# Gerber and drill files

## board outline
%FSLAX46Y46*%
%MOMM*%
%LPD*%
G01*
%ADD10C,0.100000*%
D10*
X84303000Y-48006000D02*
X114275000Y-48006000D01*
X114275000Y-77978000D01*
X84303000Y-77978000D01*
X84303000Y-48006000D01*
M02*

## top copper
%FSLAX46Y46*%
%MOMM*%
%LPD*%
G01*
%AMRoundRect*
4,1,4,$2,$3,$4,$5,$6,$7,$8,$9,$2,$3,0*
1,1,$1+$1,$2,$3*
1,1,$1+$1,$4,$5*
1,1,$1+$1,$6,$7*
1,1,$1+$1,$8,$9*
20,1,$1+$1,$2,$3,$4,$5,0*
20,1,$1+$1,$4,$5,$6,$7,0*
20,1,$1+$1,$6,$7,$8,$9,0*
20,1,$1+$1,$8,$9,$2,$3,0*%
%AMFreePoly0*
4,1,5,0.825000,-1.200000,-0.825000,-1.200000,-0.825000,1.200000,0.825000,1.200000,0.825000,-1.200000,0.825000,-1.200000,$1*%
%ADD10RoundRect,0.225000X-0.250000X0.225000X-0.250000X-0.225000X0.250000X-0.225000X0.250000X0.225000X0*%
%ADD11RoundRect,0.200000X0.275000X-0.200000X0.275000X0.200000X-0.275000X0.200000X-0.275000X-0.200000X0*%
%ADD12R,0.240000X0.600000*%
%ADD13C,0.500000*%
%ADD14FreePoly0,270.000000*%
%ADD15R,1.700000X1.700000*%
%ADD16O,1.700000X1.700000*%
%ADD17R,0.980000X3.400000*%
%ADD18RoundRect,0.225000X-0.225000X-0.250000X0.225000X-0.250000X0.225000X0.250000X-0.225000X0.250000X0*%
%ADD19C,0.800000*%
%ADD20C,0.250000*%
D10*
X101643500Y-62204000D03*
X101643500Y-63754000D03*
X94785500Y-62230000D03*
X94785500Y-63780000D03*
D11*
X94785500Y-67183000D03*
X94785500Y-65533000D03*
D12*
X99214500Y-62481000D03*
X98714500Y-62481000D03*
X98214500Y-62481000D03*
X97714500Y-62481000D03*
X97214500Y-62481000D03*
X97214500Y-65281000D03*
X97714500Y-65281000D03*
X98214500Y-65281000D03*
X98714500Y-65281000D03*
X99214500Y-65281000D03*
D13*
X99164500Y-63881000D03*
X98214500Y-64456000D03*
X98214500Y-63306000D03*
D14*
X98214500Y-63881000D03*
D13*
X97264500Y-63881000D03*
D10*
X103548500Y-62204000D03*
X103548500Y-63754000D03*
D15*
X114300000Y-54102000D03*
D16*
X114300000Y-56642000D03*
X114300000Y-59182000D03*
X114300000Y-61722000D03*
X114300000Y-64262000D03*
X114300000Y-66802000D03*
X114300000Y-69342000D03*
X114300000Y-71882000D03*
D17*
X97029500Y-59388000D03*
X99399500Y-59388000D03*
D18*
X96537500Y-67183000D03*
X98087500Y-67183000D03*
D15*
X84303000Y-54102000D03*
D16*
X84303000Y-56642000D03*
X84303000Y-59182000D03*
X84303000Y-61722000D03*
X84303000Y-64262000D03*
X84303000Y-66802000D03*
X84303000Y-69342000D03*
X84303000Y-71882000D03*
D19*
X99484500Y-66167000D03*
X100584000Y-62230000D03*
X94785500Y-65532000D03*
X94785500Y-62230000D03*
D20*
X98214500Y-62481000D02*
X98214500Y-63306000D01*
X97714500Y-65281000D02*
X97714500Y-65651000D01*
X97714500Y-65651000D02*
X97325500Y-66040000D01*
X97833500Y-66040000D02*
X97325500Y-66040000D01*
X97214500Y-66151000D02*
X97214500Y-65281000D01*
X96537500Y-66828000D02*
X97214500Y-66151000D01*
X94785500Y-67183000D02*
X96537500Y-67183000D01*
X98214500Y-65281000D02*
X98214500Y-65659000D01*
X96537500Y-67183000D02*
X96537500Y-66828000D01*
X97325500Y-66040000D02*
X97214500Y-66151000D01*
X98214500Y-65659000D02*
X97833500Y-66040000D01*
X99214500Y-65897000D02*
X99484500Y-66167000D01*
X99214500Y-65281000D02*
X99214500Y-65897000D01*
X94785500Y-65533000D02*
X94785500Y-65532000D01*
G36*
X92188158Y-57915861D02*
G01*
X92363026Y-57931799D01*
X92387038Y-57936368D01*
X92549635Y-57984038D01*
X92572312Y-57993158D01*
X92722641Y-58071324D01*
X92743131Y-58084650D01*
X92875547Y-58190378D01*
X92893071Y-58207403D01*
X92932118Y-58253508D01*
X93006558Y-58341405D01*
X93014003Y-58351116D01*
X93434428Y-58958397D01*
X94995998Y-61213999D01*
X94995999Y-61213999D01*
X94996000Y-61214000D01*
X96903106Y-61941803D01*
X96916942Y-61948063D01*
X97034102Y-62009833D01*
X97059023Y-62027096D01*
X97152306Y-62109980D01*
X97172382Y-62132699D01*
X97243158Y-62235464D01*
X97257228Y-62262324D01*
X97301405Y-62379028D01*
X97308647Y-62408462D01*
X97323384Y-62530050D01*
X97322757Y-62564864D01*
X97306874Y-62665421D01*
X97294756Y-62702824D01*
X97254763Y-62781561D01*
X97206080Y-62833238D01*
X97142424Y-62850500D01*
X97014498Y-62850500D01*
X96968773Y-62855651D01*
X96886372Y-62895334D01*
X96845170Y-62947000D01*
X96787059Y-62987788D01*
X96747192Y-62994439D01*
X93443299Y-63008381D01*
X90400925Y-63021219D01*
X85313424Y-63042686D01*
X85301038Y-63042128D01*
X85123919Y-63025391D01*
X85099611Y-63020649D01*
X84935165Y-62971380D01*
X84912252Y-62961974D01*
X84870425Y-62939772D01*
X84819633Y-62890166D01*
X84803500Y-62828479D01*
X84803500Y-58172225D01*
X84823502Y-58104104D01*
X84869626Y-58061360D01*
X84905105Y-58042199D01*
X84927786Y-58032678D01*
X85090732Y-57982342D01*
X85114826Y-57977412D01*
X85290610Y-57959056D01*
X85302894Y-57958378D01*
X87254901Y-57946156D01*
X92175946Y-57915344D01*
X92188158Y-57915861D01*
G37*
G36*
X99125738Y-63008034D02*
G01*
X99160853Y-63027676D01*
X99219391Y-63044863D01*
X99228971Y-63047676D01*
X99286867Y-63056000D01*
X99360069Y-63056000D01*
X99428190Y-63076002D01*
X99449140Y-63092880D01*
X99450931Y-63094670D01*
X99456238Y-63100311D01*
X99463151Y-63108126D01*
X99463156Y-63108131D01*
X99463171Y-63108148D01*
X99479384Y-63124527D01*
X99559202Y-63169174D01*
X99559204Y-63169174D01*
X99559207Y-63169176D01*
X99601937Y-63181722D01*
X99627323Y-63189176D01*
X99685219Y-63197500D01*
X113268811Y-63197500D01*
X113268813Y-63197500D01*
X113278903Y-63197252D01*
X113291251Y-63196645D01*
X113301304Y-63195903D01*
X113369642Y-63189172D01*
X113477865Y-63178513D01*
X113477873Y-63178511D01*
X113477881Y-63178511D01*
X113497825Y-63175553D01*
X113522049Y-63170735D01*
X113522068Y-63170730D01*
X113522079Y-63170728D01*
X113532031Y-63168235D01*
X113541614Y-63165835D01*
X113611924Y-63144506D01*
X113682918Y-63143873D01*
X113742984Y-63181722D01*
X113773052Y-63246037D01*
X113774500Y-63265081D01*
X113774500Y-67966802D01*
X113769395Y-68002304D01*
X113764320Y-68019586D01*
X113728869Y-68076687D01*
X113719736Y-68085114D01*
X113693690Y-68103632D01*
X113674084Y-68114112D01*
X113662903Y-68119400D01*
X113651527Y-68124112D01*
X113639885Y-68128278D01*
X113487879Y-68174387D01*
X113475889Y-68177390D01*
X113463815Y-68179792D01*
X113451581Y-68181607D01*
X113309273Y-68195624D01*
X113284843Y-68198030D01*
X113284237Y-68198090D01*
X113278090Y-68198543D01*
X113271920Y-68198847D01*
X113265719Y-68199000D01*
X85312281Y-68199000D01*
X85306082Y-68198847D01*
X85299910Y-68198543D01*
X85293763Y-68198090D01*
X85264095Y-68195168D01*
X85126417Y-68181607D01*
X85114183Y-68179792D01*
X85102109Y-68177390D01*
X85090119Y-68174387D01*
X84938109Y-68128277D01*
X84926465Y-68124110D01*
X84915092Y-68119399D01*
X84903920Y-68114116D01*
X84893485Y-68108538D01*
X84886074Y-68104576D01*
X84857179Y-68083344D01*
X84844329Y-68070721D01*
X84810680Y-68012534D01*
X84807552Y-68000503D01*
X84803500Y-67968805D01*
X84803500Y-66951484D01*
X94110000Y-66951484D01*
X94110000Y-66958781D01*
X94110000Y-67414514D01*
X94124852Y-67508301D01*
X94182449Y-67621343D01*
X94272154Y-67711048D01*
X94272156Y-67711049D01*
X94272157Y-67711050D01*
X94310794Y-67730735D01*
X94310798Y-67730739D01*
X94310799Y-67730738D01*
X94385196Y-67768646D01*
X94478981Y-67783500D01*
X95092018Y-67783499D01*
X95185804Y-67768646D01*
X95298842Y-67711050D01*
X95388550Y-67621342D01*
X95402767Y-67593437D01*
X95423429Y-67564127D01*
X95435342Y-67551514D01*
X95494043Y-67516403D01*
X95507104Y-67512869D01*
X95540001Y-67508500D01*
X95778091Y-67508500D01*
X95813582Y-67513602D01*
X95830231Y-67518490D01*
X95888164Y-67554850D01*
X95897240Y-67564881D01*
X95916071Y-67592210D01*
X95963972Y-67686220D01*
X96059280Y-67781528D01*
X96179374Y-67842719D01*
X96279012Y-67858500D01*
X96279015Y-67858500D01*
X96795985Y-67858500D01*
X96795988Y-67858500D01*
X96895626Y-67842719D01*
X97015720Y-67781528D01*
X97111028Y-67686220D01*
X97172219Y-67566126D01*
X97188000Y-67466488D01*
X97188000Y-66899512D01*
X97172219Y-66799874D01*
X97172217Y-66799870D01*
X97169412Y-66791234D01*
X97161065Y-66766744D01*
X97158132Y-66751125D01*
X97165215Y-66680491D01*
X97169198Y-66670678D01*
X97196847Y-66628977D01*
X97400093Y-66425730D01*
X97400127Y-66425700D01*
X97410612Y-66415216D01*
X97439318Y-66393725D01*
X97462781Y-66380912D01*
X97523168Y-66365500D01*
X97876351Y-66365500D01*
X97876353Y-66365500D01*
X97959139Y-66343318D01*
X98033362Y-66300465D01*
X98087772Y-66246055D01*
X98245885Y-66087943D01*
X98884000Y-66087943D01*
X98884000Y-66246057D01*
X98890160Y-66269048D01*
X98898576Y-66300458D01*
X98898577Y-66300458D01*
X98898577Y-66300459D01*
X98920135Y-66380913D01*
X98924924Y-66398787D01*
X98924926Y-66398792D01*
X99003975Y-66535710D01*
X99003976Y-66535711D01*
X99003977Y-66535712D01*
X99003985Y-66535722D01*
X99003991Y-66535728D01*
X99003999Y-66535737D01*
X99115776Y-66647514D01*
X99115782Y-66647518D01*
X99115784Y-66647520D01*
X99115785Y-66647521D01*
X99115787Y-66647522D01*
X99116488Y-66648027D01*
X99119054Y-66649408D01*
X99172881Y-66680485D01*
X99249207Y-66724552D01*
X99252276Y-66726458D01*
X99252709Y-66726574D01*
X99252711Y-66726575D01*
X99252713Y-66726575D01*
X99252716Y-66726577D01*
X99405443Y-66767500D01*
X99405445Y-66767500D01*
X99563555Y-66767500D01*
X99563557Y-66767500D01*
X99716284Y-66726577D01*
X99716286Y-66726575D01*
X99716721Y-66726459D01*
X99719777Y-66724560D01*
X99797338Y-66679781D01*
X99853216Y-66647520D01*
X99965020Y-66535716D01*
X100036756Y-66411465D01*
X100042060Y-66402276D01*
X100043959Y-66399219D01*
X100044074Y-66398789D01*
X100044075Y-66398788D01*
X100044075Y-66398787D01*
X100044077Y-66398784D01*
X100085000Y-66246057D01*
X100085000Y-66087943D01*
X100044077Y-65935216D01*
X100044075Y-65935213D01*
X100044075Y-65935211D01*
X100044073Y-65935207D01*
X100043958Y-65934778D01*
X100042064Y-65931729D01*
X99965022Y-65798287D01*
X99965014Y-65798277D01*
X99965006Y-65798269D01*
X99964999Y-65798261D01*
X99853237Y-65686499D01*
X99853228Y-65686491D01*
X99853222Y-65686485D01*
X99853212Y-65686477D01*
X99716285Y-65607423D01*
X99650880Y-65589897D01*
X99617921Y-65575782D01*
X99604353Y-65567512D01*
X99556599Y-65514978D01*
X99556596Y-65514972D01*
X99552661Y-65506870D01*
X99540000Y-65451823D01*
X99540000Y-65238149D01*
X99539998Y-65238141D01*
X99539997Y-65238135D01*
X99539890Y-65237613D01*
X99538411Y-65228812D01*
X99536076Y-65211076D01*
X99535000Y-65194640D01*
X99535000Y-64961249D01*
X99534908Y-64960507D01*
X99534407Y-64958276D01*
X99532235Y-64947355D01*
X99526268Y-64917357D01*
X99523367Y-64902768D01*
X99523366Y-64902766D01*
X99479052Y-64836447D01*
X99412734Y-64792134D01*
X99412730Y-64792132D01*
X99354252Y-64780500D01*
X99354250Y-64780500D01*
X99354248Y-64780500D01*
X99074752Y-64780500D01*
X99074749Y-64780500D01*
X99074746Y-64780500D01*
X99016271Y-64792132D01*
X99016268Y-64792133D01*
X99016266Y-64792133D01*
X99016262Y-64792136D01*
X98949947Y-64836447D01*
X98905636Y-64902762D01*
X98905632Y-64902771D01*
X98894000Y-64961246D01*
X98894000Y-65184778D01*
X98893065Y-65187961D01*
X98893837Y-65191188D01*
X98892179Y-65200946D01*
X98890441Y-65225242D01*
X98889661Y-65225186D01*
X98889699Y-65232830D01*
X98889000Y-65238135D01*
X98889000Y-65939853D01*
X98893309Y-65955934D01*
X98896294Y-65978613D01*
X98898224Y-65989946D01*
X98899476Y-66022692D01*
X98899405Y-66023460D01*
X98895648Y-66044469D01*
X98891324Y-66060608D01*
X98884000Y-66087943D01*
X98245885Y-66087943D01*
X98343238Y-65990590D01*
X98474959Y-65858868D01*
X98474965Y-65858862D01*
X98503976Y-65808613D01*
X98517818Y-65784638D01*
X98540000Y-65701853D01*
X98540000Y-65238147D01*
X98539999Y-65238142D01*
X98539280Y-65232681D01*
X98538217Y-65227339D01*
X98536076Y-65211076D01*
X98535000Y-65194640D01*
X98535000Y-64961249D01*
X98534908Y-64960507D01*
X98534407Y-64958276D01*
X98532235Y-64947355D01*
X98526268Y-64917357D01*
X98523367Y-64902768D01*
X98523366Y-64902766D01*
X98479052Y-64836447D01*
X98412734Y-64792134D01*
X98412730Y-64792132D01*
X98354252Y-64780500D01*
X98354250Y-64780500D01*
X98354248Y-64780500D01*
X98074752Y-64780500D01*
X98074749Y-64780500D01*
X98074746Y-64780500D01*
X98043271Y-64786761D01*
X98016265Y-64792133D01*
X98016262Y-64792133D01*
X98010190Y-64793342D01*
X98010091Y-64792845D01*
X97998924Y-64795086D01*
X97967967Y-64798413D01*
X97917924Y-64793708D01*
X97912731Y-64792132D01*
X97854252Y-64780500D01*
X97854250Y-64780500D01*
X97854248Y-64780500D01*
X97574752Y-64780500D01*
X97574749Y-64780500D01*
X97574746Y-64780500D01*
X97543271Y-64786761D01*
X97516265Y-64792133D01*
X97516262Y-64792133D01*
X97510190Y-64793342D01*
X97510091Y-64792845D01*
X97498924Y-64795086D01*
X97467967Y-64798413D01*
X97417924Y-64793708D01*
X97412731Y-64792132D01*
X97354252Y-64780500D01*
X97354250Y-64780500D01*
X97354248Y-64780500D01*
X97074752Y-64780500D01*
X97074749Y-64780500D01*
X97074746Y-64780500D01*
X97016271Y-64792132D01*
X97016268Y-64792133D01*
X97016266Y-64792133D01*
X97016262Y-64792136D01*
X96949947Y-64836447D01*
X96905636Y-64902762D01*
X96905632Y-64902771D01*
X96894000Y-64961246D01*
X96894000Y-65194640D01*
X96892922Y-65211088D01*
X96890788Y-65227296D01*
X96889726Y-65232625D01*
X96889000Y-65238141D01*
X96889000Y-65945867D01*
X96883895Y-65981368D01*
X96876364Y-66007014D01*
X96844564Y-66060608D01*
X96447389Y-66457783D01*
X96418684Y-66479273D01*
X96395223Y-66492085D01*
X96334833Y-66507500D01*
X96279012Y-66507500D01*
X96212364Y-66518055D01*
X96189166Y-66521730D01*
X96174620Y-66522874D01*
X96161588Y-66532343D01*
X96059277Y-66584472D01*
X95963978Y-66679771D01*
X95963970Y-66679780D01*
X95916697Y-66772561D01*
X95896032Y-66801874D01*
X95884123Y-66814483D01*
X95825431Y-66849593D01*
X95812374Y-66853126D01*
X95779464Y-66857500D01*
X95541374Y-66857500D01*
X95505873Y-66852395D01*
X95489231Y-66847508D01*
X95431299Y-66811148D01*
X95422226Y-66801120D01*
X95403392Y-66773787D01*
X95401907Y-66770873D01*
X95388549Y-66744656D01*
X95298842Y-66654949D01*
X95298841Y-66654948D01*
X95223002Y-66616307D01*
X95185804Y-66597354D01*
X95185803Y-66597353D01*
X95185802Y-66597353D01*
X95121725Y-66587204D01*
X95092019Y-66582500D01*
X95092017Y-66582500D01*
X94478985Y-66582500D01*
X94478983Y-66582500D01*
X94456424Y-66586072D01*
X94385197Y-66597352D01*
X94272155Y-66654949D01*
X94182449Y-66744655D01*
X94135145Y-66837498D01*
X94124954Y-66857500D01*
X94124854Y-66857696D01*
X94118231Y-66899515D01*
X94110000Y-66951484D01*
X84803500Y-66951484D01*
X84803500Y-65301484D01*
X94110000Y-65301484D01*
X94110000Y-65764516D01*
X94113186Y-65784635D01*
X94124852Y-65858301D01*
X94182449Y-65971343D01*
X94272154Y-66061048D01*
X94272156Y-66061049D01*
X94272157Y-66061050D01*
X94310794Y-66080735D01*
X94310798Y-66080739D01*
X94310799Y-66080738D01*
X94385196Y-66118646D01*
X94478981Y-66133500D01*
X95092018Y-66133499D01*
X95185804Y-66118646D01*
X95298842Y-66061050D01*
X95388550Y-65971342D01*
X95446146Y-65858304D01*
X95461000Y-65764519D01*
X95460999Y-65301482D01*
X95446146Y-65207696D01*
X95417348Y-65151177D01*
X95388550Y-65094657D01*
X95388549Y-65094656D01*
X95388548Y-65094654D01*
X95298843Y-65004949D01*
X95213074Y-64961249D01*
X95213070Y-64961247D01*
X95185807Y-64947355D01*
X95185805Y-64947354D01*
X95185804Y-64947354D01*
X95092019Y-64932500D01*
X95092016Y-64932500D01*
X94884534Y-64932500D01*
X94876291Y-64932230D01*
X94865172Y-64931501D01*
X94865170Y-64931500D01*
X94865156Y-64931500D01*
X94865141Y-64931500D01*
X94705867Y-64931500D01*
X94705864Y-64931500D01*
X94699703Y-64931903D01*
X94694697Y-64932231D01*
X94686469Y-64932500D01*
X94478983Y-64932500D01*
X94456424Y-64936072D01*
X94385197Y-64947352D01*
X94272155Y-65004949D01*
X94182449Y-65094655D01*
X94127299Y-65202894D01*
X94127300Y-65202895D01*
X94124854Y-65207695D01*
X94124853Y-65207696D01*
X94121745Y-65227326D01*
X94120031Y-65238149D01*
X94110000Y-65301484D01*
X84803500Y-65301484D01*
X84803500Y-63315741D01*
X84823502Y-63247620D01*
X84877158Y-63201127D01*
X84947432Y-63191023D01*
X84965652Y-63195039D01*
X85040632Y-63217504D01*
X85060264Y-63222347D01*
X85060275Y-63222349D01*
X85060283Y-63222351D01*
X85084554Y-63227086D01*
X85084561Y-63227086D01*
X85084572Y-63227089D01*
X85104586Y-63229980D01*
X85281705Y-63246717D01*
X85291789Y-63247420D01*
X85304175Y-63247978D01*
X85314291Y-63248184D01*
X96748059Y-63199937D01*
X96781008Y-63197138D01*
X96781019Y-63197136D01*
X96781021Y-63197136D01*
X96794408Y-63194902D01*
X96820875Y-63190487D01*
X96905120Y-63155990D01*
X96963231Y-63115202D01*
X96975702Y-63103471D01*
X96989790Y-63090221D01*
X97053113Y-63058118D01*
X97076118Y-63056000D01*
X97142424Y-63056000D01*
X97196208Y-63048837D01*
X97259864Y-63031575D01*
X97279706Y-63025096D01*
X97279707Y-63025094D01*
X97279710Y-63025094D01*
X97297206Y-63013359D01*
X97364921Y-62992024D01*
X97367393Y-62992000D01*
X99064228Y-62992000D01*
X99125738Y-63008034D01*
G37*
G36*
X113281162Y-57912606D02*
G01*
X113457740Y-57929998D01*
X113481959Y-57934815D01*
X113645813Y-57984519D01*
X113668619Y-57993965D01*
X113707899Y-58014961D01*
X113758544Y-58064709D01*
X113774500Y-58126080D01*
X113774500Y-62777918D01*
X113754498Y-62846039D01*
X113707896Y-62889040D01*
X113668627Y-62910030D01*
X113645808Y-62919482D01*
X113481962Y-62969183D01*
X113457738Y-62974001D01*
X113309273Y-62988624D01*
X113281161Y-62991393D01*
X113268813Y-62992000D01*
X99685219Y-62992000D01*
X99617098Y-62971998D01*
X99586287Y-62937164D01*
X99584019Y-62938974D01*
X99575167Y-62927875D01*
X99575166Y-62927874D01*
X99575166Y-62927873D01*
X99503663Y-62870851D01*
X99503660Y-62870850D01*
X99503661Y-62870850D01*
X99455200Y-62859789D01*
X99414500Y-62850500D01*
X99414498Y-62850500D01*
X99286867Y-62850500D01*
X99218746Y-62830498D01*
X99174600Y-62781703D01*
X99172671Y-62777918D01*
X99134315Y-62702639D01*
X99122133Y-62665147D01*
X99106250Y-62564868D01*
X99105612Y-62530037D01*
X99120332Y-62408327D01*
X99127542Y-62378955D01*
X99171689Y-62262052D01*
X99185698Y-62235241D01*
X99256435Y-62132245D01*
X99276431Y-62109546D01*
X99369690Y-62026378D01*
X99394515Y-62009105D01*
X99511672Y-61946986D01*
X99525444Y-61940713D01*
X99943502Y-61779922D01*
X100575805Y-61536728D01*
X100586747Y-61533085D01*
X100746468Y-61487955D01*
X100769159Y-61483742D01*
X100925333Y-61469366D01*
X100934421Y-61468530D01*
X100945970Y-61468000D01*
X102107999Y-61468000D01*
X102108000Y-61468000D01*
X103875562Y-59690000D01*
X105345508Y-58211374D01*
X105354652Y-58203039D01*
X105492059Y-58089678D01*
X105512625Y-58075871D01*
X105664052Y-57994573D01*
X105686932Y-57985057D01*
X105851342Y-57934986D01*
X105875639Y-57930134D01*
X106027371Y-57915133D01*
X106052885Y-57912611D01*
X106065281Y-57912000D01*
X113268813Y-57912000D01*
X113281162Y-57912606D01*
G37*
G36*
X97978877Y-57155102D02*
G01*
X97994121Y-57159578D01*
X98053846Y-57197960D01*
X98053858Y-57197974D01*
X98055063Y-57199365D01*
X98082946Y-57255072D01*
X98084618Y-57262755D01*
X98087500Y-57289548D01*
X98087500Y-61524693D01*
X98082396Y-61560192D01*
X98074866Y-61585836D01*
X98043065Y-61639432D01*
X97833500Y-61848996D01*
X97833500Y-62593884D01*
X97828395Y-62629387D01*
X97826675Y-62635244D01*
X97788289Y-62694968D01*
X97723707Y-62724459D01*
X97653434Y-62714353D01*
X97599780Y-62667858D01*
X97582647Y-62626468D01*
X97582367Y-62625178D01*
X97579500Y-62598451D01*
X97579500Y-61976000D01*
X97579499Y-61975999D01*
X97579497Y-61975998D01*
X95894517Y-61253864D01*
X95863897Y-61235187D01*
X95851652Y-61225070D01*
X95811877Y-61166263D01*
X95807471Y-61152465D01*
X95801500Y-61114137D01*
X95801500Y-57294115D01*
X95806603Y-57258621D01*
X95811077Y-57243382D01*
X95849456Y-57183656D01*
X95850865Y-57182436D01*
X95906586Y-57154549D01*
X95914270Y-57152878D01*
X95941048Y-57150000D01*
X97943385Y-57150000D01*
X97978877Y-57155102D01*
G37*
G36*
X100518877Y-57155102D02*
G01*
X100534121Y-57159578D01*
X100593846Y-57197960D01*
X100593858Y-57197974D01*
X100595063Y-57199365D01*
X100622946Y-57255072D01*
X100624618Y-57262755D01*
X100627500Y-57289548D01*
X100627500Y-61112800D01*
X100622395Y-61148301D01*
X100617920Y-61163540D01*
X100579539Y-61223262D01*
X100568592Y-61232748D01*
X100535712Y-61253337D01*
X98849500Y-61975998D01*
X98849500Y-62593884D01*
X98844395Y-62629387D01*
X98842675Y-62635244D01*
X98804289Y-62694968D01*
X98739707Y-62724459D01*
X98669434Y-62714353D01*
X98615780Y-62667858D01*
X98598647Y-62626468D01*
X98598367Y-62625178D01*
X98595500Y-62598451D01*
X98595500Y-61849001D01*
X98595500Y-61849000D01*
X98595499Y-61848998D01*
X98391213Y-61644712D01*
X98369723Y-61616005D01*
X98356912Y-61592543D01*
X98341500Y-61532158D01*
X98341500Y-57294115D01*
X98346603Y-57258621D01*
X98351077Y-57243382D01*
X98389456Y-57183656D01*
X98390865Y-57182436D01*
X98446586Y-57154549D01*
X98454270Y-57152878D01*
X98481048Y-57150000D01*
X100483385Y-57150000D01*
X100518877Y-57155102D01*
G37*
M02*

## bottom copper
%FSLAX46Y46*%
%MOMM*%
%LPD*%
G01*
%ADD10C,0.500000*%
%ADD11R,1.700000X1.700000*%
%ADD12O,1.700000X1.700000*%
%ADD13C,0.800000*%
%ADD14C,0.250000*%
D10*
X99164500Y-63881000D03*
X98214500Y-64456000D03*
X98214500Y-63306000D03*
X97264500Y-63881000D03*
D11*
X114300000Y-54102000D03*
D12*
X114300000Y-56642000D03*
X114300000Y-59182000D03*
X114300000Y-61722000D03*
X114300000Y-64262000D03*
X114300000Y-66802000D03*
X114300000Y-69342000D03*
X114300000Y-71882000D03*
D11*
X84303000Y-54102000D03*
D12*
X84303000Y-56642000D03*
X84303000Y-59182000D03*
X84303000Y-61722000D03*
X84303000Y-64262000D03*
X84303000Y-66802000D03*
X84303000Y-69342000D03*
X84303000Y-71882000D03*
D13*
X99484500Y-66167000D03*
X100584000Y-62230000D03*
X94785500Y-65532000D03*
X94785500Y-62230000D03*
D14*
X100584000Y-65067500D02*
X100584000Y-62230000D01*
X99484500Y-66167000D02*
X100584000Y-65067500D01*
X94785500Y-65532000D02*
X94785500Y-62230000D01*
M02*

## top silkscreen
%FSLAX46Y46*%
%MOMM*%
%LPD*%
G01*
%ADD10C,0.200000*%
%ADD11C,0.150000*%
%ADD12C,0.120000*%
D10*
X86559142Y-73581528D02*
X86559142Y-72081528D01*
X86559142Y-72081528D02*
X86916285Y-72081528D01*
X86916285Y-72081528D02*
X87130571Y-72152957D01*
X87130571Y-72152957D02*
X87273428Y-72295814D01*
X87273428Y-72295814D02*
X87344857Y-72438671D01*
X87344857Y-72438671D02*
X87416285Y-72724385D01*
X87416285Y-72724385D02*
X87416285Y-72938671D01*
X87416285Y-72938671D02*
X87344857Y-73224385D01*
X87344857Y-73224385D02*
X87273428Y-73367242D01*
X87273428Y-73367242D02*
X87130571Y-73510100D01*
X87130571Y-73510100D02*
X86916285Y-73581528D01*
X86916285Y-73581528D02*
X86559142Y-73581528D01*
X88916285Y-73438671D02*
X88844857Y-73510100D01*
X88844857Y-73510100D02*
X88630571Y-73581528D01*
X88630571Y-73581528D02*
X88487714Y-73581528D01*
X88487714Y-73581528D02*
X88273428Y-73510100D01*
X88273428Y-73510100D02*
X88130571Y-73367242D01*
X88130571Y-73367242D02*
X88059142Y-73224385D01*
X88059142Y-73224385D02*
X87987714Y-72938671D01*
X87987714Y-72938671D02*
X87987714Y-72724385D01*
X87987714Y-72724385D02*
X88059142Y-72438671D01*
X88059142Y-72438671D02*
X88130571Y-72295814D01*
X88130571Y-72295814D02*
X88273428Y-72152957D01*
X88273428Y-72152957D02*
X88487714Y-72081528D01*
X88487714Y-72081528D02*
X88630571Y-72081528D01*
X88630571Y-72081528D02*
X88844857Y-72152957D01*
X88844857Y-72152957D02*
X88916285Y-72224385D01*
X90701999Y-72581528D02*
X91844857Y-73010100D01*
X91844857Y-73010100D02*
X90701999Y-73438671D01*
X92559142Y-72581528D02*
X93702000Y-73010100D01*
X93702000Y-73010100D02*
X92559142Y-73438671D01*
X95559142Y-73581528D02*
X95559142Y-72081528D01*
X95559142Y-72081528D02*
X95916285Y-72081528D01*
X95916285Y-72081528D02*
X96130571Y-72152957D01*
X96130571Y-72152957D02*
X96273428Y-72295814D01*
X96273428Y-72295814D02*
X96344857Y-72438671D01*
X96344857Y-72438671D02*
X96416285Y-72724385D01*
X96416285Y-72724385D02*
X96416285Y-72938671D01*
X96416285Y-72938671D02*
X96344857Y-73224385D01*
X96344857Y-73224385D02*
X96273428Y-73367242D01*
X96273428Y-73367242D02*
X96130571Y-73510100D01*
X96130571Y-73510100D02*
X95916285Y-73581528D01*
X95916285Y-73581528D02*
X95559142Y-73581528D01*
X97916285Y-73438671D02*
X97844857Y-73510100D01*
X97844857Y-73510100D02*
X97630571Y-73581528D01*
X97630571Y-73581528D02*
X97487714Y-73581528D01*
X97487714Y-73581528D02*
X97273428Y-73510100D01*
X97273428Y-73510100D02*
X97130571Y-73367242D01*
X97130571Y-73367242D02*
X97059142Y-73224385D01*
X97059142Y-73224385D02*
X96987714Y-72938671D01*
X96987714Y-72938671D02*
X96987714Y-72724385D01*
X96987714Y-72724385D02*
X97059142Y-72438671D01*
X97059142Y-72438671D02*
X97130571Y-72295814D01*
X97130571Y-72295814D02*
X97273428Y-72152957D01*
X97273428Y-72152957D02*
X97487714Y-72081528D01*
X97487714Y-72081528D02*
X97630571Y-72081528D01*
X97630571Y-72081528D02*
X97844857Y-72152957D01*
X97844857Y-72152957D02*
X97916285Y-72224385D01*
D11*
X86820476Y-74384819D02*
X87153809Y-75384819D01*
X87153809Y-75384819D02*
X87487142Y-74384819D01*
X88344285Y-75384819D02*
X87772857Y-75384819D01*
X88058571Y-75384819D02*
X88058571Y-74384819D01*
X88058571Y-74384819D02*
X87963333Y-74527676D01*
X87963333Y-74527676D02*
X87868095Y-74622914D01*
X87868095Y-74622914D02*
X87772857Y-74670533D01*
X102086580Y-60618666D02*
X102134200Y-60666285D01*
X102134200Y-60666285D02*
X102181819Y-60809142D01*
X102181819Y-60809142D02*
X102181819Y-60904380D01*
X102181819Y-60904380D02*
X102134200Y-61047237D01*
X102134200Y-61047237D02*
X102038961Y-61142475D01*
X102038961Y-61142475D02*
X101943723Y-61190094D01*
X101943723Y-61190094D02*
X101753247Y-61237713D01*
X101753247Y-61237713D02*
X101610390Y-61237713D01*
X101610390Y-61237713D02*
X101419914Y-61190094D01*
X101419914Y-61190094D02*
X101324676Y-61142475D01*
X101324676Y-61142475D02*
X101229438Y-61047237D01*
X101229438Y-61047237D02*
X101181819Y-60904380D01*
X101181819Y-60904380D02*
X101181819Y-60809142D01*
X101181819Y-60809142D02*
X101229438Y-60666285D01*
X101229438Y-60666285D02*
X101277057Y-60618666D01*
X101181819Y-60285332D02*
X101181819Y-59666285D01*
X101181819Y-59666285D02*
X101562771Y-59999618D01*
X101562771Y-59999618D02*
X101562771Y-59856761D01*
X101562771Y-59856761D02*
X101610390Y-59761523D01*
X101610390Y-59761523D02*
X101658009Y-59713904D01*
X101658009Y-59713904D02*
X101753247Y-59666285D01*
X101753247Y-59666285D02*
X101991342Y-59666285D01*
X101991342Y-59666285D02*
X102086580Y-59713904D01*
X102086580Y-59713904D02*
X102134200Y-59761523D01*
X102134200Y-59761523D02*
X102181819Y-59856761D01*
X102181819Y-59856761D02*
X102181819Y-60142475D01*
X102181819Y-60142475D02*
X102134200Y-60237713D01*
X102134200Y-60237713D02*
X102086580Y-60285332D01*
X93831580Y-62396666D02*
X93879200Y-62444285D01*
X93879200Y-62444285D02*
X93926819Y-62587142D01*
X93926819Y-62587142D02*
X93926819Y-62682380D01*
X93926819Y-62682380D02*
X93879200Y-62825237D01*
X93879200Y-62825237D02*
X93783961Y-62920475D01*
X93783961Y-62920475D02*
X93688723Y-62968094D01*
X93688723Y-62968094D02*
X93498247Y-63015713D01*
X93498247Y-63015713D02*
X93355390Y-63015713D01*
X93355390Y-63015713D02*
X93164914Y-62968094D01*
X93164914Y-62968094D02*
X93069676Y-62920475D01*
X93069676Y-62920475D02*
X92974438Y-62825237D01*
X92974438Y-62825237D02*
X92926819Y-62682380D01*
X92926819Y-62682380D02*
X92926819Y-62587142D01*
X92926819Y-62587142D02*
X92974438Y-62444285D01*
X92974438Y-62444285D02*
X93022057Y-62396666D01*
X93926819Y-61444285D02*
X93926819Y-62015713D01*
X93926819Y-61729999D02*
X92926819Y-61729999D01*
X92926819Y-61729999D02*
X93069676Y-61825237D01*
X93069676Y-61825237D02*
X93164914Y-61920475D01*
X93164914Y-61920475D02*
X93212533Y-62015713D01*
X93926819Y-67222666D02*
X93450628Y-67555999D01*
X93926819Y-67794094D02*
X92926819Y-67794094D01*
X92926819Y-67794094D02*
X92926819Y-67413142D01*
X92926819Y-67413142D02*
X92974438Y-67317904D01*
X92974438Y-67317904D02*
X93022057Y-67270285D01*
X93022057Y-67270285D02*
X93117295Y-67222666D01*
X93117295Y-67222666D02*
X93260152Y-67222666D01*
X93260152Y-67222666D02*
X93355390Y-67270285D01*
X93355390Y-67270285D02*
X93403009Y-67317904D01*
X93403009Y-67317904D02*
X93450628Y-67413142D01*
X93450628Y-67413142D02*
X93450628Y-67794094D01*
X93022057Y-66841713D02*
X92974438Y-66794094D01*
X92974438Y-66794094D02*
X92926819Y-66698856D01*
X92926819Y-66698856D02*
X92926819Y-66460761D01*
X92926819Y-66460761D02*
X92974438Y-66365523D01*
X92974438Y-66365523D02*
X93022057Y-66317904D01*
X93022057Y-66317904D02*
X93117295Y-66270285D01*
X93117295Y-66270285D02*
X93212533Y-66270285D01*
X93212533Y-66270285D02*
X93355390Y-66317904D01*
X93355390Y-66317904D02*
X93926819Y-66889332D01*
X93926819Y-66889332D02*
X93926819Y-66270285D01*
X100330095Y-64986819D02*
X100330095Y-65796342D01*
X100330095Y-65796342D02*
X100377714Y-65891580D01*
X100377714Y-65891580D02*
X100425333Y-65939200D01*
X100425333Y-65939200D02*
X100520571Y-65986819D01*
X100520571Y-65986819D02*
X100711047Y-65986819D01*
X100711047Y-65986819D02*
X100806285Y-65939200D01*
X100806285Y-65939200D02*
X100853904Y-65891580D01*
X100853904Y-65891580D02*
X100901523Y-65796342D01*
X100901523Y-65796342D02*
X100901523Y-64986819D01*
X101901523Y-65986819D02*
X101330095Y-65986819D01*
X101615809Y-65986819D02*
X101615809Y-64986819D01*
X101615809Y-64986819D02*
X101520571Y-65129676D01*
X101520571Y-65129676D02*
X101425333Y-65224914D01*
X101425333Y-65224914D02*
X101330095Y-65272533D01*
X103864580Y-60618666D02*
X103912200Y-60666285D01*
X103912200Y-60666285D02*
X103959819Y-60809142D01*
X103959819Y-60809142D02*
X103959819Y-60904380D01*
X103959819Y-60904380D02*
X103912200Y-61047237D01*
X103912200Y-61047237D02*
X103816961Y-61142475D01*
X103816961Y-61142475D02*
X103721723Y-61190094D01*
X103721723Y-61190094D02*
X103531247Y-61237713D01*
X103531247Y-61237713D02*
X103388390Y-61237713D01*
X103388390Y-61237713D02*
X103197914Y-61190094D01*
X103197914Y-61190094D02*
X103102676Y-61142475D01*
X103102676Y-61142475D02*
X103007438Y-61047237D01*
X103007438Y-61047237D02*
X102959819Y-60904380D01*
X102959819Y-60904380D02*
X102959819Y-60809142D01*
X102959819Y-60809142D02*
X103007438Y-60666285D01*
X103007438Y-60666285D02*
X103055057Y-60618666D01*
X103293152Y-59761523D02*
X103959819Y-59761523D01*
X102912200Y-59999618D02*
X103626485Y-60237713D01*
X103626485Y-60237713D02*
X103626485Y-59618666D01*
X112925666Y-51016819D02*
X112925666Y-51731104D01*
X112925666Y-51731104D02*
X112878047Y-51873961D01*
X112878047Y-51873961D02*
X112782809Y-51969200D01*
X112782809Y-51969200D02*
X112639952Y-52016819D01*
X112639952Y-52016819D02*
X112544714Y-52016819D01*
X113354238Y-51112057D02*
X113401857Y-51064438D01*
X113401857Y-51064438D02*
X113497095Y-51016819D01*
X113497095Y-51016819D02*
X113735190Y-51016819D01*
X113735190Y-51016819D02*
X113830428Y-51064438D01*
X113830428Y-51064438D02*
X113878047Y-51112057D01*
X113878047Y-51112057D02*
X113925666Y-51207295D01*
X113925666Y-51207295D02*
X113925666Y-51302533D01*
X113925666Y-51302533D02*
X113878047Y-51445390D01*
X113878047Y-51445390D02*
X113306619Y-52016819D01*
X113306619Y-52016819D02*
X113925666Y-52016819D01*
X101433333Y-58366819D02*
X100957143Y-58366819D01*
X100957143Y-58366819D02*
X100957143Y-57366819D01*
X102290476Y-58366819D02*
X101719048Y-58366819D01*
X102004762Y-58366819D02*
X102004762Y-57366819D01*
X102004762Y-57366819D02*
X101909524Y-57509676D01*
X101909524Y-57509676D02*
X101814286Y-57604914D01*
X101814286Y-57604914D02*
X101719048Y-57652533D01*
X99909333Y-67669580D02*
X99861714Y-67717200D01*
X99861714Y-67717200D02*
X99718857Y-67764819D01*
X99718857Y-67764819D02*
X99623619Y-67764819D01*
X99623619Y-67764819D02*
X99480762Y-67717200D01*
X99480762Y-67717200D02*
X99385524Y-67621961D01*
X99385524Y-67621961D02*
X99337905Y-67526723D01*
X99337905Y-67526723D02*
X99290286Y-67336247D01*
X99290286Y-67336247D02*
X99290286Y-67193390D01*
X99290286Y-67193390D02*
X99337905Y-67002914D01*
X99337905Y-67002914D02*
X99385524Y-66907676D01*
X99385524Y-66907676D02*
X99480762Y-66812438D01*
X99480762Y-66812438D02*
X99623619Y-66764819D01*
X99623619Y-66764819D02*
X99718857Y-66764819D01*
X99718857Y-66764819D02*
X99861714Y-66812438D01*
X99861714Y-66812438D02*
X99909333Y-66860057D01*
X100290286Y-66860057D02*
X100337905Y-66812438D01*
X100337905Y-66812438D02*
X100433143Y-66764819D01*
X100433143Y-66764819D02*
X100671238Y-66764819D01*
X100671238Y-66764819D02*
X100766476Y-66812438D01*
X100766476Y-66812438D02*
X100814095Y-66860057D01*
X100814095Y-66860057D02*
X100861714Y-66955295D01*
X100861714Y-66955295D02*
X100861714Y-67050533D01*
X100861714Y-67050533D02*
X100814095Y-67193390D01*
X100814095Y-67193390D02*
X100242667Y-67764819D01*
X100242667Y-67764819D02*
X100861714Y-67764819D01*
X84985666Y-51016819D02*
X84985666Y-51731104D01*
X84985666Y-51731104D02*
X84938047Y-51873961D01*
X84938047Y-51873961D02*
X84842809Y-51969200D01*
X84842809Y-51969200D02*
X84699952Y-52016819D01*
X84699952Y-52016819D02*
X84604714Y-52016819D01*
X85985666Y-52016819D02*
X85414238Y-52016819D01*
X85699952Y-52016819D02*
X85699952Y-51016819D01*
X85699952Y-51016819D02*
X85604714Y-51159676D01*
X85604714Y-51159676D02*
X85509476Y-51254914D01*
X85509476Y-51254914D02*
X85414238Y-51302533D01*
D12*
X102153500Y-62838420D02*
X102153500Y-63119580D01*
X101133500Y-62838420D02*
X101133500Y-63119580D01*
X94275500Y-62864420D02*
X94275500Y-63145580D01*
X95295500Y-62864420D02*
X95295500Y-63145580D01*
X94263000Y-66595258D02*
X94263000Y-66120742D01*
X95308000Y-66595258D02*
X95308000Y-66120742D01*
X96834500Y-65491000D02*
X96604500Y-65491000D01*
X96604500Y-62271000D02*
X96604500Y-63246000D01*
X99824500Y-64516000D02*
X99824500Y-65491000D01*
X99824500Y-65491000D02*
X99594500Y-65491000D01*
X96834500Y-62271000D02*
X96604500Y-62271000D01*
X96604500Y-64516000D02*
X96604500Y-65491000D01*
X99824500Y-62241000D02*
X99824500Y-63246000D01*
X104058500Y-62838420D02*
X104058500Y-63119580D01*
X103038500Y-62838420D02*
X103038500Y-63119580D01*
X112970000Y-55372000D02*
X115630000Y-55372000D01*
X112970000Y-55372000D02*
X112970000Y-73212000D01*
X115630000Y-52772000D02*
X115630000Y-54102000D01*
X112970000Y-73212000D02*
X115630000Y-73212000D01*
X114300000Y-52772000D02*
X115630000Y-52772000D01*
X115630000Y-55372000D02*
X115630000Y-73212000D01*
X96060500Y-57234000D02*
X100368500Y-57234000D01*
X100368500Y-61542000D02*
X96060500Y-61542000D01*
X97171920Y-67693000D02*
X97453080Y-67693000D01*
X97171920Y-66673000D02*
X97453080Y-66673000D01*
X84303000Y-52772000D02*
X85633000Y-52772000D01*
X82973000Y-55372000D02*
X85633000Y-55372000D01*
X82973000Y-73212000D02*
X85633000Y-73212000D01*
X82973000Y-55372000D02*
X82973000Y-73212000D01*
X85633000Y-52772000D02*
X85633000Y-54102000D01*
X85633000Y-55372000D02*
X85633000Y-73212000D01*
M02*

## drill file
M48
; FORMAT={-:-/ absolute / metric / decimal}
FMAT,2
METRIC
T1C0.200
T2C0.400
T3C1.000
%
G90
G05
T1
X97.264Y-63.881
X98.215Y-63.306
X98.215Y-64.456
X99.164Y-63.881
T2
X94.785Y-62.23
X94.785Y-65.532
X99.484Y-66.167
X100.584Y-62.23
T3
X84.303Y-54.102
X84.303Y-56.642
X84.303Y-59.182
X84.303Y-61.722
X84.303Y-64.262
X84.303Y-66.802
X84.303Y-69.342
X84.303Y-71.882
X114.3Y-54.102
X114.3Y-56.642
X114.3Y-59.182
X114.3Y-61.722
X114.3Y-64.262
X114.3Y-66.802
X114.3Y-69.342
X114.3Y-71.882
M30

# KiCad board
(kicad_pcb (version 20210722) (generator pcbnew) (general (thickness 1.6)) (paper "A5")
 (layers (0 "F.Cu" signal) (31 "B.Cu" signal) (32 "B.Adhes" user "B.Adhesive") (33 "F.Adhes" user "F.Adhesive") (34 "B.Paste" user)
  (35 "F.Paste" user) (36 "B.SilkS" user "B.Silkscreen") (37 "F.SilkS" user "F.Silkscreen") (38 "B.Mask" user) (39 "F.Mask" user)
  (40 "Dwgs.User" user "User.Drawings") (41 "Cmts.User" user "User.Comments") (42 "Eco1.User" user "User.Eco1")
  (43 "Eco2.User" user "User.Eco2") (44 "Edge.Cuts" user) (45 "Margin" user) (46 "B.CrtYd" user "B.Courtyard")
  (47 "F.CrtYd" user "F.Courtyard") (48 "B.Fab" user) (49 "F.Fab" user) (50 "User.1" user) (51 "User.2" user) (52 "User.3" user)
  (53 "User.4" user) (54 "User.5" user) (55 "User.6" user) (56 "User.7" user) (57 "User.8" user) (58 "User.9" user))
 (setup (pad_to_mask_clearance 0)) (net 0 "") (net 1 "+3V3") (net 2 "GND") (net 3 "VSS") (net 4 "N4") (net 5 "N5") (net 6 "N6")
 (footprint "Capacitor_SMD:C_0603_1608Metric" (layer "F.Cu") (at 101.6435 62.979 -90)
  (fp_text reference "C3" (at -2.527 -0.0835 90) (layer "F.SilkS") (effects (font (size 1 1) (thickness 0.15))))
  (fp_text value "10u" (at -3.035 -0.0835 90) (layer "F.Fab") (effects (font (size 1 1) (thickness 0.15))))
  (fp_line (start -0.14058 -0.51) (end 0.14058 -0.51) (layer "F.SilkS") (width 0.12))
  (fp_line (start -0.14058 0.51) (end 0.14058 0.51) (layer "F.SilkS") (width 0.12))
  (pad "1" smd roundrect locked (at -0.775 0 270) (size 0.9 0.95) (layers "F.Cu" "F.Paste" "F.Mask") (roundrect_rratio 0.25) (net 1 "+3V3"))
  (pad "2" smd roundrect locked (at 0.775 0 270) (size 0.9 0.95) (layers "F.Cu" "F.Paste" "F.Mask") (roundrect_rratio 0.25) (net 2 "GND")))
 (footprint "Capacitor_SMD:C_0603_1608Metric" (layer "F.Cu") (at 94.7855 63.005 -90)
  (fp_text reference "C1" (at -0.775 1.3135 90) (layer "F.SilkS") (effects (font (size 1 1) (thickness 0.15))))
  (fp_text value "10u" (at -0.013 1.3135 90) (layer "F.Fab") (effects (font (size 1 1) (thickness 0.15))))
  (fp_line (start -0.14058 0.51) (end 0.14058 0.51) (layer "F.SilkS") (width 0.12))
  (fp_line (start -0.14058 -0.51) (end 0.14058 -0.51) (layer "F.SilkS") (width 0.12))
  (pad "1" smd roundrect locked (at -0.775 0 270) (size 0.9 0.95) (layers "F.Cu" "F.Paste" "F.Mask") (roundrect_rratio 0.25) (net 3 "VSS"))
  (pad "2" smd roundrect locked (at 0.775 0 270) (size 0.9 0.95) (layers "F.Cu" "F.Paste" "F.Mask") (roundrect_rratio 0.25) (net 2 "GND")))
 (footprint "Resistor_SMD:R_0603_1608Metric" (layer "F.Cu") (at 94.7855 66.358 90)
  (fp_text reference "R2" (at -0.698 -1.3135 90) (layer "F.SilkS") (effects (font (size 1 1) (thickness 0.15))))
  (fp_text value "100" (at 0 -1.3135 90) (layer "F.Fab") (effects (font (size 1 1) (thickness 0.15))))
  (fp_line (start -0.237258 -0.5225) (end 0.237258 -0.5225) (layer "F.SilkS") (width 0.12))
  (fp_line (start -0.237258 0.5225) (end 0.237258 0.5225) (layer "F.SilkS") (width 0.12))
  (pad "1" smd roundrect locked (at -0.825 0 90) (size 0.8 0.95) (layers "F.Cu" "F.Paste" "F.Mask") (roundrect_rratio 0.25) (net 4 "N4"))
  (pad "2" smd roundrect locked (at 0.825 0 90) (size 0.8 0.95) (layers "F.Cu" "F.Paste" "F.Mask") (roundrect_rratio 0.25) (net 3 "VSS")))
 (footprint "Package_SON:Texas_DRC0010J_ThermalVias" (layer "F.Cu") (at 98.2145 63.881 -90)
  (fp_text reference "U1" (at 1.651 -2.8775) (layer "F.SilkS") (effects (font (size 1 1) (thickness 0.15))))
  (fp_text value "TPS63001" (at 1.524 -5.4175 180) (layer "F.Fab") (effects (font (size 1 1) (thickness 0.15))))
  (fp_line (start 1.61 1.38) (end 1.61 1.61) (layer "F.SilkS") (width 0.12))
  (fp_line (start -1.61 1.61) (end -0.635 1.61) (layer "F.SilkS") (width 0.12))
  (fp_line (start 0.635 -1.61) (end 1.61 -1.61) (layer "F.SilkS") (width 0.12))
  (fp_line (start 1.61 -1.61) (end 1.61 -1.38) (layer "F.SilkS") (width 0.12))
  (fp_line (start -1.61 1.38) (end -1.61 1.61) (layer "F.SilkS") (width 0.12))
  (fp_line (start 0.635 1.61) (end 1.61 1.61) (layer "F.SilkS") (width 0.12))
  (fp_line (start -1.64 -1.61) (end -0.635 -1.61) (layer "F.SilkS") (width 0.12))
  (pad "" smd roundrect locked (at 0 -0.63 270) (size 1.5 1.06) (layers "F.Paste") (roundrect_rratio 0.1) (zone_connect 0))
  (pad "" smd roundrect locked (at 0.25 1.53 270) (size 0.25 0.34) (layers "F.Paste") (roundrect_rratio 0.1) (zone_connect 0))
  (pad "" smd roundrect locked (at -0.25 -1.53 270) (size 0.25 0.34) (layers "F.Paste") (roundrect_rratio 0.1) (zone_connect 0))
  (pad "" smd roundrect locked (at 0 0.63 270) (size 1.5 1.06) (layers "F.Paste") (roundrect_rratio 0.1) (zone_connect 0))
  (pad "" smd roundrect locked (at -0.25 1.53 270) (size 0.25 0.34) (layers "F.Paste") (roundrect_rratio 0.1) (zone_connect 0))
  (pad "" smd roundrect locked (at 0.25 -1.53 270) (size 0.25 0.34) (layers "F.Paste") (roundrect_rratio 0.1) (zone_connect 0))
  (pad "1" smd rect locked (at -1.4 -1 270) (size 0.6 0.24) (layers "F.Cu" "F.Paste" "F.Mask") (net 1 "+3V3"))
  (pad "2" smd rect locked (at -1.4 -0.5 270) (size 0.6 0.24) (layers "F.Cu" "F.Paste" "F.Mask") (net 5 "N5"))
  (pad "3" smd rect locked (at -1.4 0 270) (size 0.6 0.24) (layers "F.Cu" "F.Paste" "F.Mask") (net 2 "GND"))
  (pad "4" smd rect locked (at -1.4 0.5 270) (size 0.6 0.24) (layers "F.Cu" "F.Paste" "F.Mask") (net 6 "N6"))
  (pad "5" smd rect locked (at -1.4 1 270) (size 0.6 0.24) (layers "F.Cu" "F.Paste" "F.Mask") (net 3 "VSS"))
  (pad "6" smd rect locked (at 1.4 1 270) (size 0.6 0.24) (layers "F.Cu" "F.Paste" "F.Mask") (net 4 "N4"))
  (pad "7" smd rect locked (at 1.4 0.5 270) (size 0.6 0.24) (layers "F.Cu" "F.Paste" "F.Mask") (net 4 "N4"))
  (pad "8" smd rect locked (at 1.4 0 270) (size 0.6 0.24) (layers "F.Cu" "F.Paste" "F.Mask") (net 4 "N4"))
  (pad "9" smd rect locked (at 1.4 -0.5 270) (size 0.6 0.24) (layers "F.Cu" "F.Paste" "F.Mask") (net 2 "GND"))
  (pad "10" smd rect locked (at 1.4 -1 270) (size 0.6 0.24) (layers "F.Cu" "F.Paste" "F.Mask") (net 1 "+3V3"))
  (pad "11" thru_hole circle locked (at 0 -0.95 270) (size 0.5 0.5) (drill 0.2) (layers *.Cu) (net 2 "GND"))
  (pad "11" thru_hole circle locked (at 0.575 0 270) (size 0.5 0.5) (drill 0.2) (layers *.Cu) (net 2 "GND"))
  (pad "11" thru_hole circle locked (at -0.575 0 270) (size 0.5 0.5) (drill 0.2) (layers *.Cu) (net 2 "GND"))
  (pad "11" smd custom locked (at 0 0 270) (size 1.65 2.4) (layers "F.Cu" "F.Mask") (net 2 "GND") (zone_connect 2)
   (options (clearance outline) (anchor rect)) (primitives))
  (pad "11" thru_hole circle locked (at 0 0.95 270) (size 0.5 0.5) (drill 0.2) (layers *.Cu) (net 2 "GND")))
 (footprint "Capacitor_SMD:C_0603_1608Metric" (layer "F.Cu") (at 103.5485 62.979 -90)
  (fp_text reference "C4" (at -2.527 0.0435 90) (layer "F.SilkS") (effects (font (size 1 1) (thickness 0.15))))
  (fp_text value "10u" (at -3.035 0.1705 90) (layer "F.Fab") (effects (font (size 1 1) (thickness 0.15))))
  (fp_line (start -0.14058 -0.51) (end 0.14058 -0.51) (layer "F.SilkS") (width 0.12))
  (fp_line (start -0.14058 0.51) (end 0.14058 0.51) (layer "F.SilkS") (width 0.12))
  (pad "1" smd roundrect locked (at -0.775 0 270) (size 0.9 0.95) (layers "F.Cu" "F.Paste" "F.Mask") (roundrect_rratio 0.25) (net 1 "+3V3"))
  (pad "2" smd roundrect locked (at 0.775 0 270) (size 0.9 0.95) (layers "F.Cu" "F.Paste" "F.Mask") (roundrect_rratio 0.25) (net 2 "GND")))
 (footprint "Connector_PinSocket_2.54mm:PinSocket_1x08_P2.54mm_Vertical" (layer "F.Cu") (at 114.3 54.102)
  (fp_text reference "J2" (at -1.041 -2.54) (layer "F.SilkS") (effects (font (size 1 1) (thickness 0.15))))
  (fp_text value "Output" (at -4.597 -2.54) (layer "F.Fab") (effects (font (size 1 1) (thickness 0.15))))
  (fp_line (start -1.33 1.27) (end 1.33 1.27) (layer "F.SilkS") (width 0.12))
  (fp_line (start -1.33 1.27) (end -1.33 19.11) (layer "F.SilkS") (width 0.12))
  (fp_line (start 1.33 -1.33) (end 1.33 0) (layer "F.SilkS") (width 0.12))
  (fp_line (start -1.33 19.11) (end 1.33 19.11) (layer "F.SilkS") (width 0.12))
  (fp_line (start 0 -1.33) (end 1.33 -1.33) (layer "F.SilkS") (width 0.12))
  (fp_line (start 1.33 1.27) (end 1.33 19.11) (layer "F.SilkS") (width 0.12))
  (pad "1" thru_hole rect locked (at 0 0) (size 1.7 1.7) (drill 1) (layers *.Cu *.Mask))
  (pad "2" thru_hole oval locked (at 0 2.54) (size 1.7 1.7) (drill 1) (layers *.Cu *.Mask))
  (pad "3" thru_hole oval locked (at 0 5.08) (size 1.7 1.7) (drill 1) (layers *.Cu *.Mask) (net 1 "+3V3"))
  (pad "4" thru_hole oval locked (at 0 7.62) (size 1.7 1.7) (drill 1) (layers *.Cu *.Mask) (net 1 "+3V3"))
  (pad "5" thru_hole oval locked (at 0 10.16) (size 1.7 1.7) (drill 1) (layers *.Cu *.Mask) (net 2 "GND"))
  (pad "6" thru_hole oval locked (at 0 12.7) (size 1.7 1.7) (drill 1) (layers *.Cu *.Mask) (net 2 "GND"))
  (pad "7" thru_hole oval locked (at 0 15.24) (size 1.7 1.7) (drill 1) (layers *.Cu *.Mask))
  (pad "8" thru_hole oval locked (at 0 17.78) (size 1.7 1.7) (drill 1) (layers *.Cu *.Mask)))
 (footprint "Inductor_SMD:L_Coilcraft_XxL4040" (layer "F.Cu") (at 98.2145 59.388)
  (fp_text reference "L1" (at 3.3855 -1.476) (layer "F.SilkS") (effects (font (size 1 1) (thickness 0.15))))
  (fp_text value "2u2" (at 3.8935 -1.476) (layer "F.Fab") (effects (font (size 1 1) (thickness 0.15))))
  (fp_line (start -2.154 -2.154) (end 2.154 -2.154) (layer "F.SilkS") (width 0.12))
  (fp_line (start 2.154 2.154) (end -2.154 2.154) (layer "F.SilkS") (width 0.12))
  (pad "1" smd rect locked (at -1.185 0) (size 0.98 3.4) (layers "F.Cu" "F.Paste" "F.Mask") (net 6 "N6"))
  (pad "2" smd rect locked (at 1.185 0) (size 0.98 3.4) (layers "F.Cu" "F.Paste" "F.Mask") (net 5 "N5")))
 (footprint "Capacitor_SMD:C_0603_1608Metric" (layer "F.Cu") (at 97.3125 67.183)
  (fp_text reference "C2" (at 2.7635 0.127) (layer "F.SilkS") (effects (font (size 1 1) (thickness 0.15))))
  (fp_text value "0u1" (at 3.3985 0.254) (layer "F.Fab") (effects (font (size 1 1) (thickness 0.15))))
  (fp_line (start -0.14058 0.51) (end 0.14058 0.51) (layer "F.SilkS") (width 0.12))
  (fp_line (start -0.14058 -0.51) (end 0.14058 -0.51) (layer "F.SilkS") (width 0.12))
  (pad "1" smd roundrect locked (at -0.775 0) (size 0.9 0.95) (layers "F.Cu" "F.Paste" "F.Mask") (roundrect_rratio 0.25) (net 4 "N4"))
  (pad "2" smd roundrect locked (at 0.775 0) (size 0.9 0.95) (layers "F.Cu" "F.Paste" "F.Mask") (roundrect_rratio 0.25) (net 2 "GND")))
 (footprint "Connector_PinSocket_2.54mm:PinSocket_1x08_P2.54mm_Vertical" (layer "F.Cu") (at 84.303 54.102)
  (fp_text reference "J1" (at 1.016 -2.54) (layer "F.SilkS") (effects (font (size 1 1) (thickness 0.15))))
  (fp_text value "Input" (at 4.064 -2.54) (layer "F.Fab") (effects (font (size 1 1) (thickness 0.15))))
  (fp_line (start 0 -1.33) (end 1.33 -1.33) (layer "F.SilkS") (width 0.12))
  (fp_line (start -1.33 1.27) (end 1.33 1.27) (layer "F.SilkS") (width 0.12))
  (fp_line (start -1.33 19.11) (end 1.33 19.11) (layer "F.SilkS") (width 0.12))
  (fp_line (start -1.33 1.27) (end -1.33 19.11) (layer "F.SilkS") (width 0.12))
  (fp_line (start 1.33 -1.33) (end 1.33 0) (layer "F.SilkS") (width 0.12))
  (fp_line (start 1.33 1.27) (end 1.33 19.11) (layer "F.SilkS") (width 0.12))
  (pad "1" thru_hole rect locked (at 0 0) (size 1.7 1.7) (drill 1) (layers *.Cu *.Mask))
  (pad "2" thru_hole oval locked (at 0 2.54) (size 1.7 1.7) (drill 1) (layers *.Cu *.Mask))
  (pad "3" thru_hole oval locked (at 0 5.08) (size 1.7 1.7) (drill 1) (layers *.Cu *.Mask) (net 3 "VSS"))
  (pad "4" thru_hole oval locked (at 0 7.62) (size 1.7 1.7) (drill 1) (layers *.Cu *.Mask) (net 3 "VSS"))
  (pad "5" thru_hole oval locked (at 0 10.16) (size 1.7 1.7) (drill 1) (layers *.Cu *.Mask) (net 2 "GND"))
  (pad "6" thru_hole oval locked (at 0 12.7) (size 1.7 1.7) (drill 1) (layers *.Cu *.Mask) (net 2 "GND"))
  (pad "7" thru_hole oval locked (at 0 15.24) (size 1.7 1.7) (drill 1) (layers *.Cu *.Mask))
  (pad "8" thru_hole oval locked (at 0 17.78) (size 1.7 1.7) (drill 1) (layers *.Cu *.Mask)))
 (gr_rect (start 84.303 48.006) (end 114.275 77.978) (layer "Edge.Cuts") (width 0.1) (fill none))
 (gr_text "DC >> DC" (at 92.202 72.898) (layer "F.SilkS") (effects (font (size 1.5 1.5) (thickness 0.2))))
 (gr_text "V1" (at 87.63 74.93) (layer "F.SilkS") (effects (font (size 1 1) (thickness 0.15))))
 (segment (start 98.2145 62.481) (end 98.2145 63.306) (width 0.25) (layer "F.Cu") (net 2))
 (segment (start 97.7145 65.281) (end 97.7145 65.651) (width 0.25) (layer "F.Cu") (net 4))
 (segment (start 97.7145 65.651) (end 97.3255 66.04) (width 0.25) (layer "F.Cu") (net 4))
 (segment (start 97.8335 66.04) (end 97.3255 66.04) (width 0.25) (layer "F.Cu") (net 4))
 (segment (start 97.2145 66.151) (end 97.2145 65.281) (width 0.25) (layer "F.Cu") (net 4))
 (segment (start 96.5375 66.828) (end 97.2145 66.151) (width 0.25) (layer "F.Cu") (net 4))
 (segment (start 94.7855 67.183) (end 96.5375 67.183) (width 0.25) (layer "F.Cu") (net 4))
 (segment (start 98.2145 65.281) (end 98.2145 65.659) (width 0.25) (layer "F.Cu") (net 4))
 (segment (start 96.5375 67.183) (end 96.5375 66.828) (width 0.25) (layer "F.Cu") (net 4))
 (segment (start 97.3255 66.04) (end 97.2145 66.151) (width 0.25) (layer "F.Cu") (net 4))
 (segment (start 98.2145 65.659) (end 97.8335 66.04) (width 0.25) (layer "F.Cu") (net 4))
 (segment (start 99.2145 65.897) (end 99.4845 66.167) (width 0.25) (layer "F.Cu") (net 1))
 (segment (start 99.2145 65.281) (end 99.2145 65.897) (width 0.25) (layer "F.Cu") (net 1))
 (via (at 99.4845 66.167) (size 0.8) (drill 0.4) (layers "F.Cu" "B.Cu") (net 1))
 (via (at 100.584 62.23) (size 0.8) (drill 0.4) (layers "F.Cu" "B.Cu") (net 1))
 (segment (start 100.584 65.0675) (end 100.584 62.23) (width 0.25) (layer "B.Cu") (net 1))
 (segment (start 99.4845 66.167) (end 100.584 65.0675) (width 0.25) (layer "B.Cu") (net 1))
 (segment (start 94.7855 65.533) (end 94.7855 65.532) (width 0.25) (layer "F.Cu") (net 3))
 (via (at 94.7855 65.532) (size 0.8) (drill 0.4) (layers "F.Cu" "B.Cu") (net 3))
 (via (at 94.7855 62.23) (size 0.8) (drill 0.4) (layers "F.Cu" "B.Cu") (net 3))
 (segment (start 94.7855 65.532) (end 94.7855 62.23) (width 0.25) (layer "B.Cu") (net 3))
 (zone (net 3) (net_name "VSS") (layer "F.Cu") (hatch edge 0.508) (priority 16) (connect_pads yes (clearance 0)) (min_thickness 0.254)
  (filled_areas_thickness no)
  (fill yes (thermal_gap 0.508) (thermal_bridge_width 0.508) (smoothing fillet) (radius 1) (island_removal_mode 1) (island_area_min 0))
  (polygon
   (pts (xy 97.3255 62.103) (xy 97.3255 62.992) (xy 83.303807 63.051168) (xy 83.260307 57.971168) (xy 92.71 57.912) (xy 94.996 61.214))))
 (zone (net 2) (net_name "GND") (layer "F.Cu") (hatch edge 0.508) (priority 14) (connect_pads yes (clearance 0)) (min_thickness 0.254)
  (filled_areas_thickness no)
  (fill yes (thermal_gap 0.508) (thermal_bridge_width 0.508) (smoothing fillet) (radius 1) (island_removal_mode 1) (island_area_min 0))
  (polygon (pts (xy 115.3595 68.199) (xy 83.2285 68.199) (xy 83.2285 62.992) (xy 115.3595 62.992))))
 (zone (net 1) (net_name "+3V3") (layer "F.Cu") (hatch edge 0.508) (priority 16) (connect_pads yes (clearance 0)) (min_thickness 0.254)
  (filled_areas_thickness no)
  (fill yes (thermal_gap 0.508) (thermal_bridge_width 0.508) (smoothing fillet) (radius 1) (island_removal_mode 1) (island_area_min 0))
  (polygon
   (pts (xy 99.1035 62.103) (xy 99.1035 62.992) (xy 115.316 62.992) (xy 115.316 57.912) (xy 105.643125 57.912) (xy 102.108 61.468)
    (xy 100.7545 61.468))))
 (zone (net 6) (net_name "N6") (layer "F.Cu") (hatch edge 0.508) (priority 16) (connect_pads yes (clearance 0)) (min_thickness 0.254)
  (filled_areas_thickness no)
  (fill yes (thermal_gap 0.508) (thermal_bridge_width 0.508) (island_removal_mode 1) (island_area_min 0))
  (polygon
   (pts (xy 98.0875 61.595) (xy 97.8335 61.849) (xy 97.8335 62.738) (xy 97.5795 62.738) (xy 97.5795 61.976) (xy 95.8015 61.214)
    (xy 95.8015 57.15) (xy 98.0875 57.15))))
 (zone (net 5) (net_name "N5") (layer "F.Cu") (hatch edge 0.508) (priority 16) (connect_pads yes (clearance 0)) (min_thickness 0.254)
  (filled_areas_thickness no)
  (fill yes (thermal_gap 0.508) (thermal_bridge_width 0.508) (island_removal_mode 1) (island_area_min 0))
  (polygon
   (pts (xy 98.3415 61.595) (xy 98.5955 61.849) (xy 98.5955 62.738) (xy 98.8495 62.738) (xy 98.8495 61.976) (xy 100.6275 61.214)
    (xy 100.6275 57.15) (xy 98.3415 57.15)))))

